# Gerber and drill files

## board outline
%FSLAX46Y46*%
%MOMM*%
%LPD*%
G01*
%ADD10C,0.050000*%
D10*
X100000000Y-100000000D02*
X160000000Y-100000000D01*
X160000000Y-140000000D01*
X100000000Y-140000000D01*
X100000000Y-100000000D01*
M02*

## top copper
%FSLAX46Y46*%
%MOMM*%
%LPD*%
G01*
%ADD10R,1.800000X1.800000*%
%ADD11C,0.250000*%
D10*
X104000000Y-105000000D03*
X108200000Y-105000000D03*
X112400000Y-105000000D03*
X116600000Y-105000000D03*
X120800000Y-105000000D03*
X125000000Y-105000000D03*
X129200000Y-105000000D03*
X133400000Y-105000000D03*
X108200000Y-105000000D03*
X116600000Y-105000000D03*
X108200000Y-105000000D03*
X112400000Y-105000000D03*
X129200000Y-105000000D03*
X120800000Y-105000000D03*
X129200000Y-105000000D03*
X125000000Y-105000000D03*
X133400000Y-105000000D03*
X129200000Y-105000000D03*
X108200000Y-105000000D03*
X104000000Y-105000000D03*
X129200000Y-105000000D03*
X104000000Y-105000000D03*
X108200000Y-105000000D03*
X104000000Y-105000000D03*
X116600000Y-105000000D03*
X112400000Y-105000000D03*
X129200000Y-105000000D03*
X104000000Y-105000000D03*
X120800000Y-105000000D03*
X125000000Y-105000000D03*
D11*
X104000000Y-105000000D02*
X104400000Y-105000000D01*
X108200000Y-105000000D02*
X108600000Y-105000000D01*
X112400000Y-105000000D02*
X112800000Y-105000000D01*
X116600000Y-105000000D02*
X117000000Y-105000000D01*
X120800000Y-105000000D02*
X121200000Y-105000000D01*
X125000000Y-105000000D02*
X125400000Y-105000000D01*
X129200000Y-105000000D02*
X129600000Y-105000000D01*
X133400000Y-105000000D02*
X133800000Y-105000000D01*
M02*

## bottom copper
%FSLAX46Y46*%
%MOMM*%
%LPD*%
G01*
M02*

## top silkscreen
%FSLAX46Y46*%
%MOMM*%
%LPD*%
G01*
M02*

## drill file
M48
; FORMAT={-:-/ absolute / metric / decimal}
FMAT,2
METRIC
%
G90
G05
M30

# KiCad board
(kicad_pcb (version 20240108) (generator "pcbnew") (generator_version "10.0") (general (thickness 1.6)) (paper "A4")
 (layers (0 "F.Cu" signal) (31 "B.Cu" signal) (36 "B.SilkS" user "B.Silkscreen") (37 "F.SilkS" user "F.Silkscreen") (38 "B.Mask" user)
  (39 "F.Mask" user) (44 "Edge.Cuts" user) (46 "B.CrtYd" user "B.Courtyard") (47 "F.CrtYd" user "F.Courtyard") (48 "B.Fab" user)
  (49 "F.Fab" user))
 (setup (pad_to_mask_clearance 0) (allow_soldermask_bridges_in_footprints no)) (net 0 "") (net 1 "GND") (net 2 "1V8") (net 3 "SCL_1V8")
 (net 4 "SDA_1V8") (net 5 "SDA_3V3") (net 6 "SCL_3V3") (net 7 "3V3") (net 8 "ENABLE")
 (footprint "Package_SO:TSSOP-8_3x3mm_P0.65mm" (layer "F.Cu") (at 100 100)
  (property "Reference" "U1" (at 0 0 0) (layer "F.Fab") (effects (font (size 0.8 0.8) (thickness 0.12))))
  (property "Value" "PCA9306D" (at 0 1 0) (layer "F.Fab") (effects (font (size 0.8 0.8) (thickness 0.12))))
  (pad "1" smd rect (at 4.000 5.000) (size 1.8 1.8) (layers "F.Cu" "F.Paste" "F.Mask") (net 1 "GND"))
  (pad "2" smd rect (at 8.200 5.000) (size 1.8 1.8) (layers "F.Cu" "F.Paste" "F.Mask") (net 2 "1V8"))
  (pad "3" smd rect (at 12.400 5.000) (size 1.8 1.8) (layers "F.Cu" "F.Paste" "F.Mask") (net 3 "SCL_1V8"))
  (pad "4" smd rect (at 16.600 5.000) (size 1.8 1.8) (layers "F.Cu" "F.Paste" "F.Mask") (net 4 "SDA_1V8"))
  (pad "5" smd rect (at 20.800 5.000) (size 1.8 1.8) (layers "F.Cu" "F.Paste" "F.Mask") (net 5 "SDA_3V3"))
  (pad "6" smd rect (at 25.000 5.000) (size 1.8 1.8) (layers "F.Cu" "F.Paste" "F.Mask") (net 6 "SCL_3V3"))
  (pad "7" smd rect (at 29.200 5.000) (size 1.8 1.8) (layers "F.Cu" "F.Paste" "F.Mask") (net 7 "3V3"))
  (pad "8" smd rect (at 33.400 5.000) (size 1.8 1.8) (layers "F.Cu" "F.Paste" "F.Mask") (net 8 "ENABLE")))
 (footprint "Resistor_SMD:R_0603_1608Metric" (layer "F.Cu") (at 100 100)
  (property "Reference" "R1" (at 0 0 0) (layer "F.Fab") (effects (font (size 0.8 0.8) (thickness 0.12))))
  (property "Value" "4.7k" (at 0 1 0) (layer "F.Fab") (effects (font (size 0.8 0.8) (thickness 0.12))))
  (pad "1" smd rect (at 8.200 5.000) (size 1.8 1.8) (layers "F.Cu" "F.Paste" "F.Mask") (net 2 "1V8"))
  (pad "2" smd rect (at 16.600 5.000) (size 1.8 1.8) (layers "F.Cu" "F.Paste" "F.Mask") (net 4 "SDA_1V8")))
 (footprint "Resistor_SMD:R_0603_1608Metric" (layer "F.Cu") (at 100 100)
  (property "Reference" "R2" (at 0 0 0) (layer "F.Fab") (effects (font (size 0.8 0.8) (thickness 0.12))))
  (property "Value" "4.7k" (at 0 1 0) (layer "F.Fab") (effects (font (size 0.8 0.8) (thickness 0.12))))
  (pad "1" smd rect (at 8.200 5.000) (size 1.8 1.8) (layers "F.Cu" "F.Paste" "F.Mask") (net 2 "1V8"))
  (pad "2" smd rect (at 12.400 5.000) (size 1.8 1.8) (layers "F.Cu" "F.Paste" "F.Mask") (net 3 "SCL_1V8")))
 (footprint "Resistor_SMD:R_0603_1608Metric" (layer "F.Cu") (at 100 100)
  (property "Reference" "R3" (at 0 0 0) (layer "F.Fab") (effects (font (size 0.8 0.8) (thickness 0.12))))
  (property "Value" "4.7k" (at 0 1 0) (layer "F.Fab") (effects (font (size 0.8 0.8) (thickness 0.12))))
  (pad "1" smd rect (at 29.200 5.000) (size 1.8 1.8) (layers "F.Cu" "F.Paste" "F.Mask") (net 7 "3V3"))
  (pad "2" smd rect (at 20.800 5.000) (size 1.8 1.8) (layers "F.Cu" "F.Paste" "F.Mask") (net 5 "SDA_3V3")))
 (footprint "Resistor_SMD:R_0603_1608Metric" (layer "F.Cu") (at 100 100)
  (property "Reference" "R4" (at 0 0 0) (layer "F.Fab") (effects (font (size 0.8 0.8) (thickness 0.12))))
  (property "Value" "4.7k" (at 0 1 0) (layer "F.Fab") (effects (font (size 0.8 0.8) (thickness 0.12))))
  (pad "1" smd rect (at 29.200 5.000) (size 1.8 1.8) (layers "F.Cu" "F.Paste" "F.Mask") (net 7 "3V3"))
  (pad "2" smd rect (at 25.000 5.000) (size 1.8 1.8) (layers "F.Cu" "F.Paste" "F.Mask") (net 6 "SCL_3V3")))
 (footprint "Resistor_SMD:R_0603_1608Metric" (layer "F.Cu") (at 100 100)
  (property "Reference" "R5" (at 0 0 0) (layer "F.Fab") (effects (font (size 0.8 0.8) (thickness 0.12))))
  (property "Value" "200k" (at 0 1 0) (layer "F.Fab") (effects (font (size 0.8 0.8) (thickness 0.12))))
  (pad "1" smd rect (at 33.400 5.000) (size 1.8 1.8) (layers "F.Cu" "F.Paste" "F.Mask") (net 8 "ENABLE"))
  (pad "2" smd rect (at 29.200 5.000) (size 1.8 1.8) (layers "F.Cu" "F.Paste" "F.Mask") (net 7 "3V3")))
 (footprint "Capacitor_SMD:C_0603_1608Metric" (layer "F.Cu") (at 100 100)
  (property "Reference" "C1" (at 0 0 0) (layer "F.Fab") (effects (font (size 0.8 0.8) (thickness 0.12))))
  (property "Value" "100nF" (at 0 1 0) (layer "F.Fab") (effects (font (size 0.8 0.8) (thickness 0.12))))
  (pad "1" smd rect (at 8.200 5.000) (size 1.8 1.8) (layers "F.Cu" "F.Paste" "F.Mask") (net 2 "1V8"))
  (pad "2" smd rect (at 4.000 5.000) (size 1.8 1.8) (layers "F.Cu" "F.Paste" "F.Mask") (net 1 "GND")))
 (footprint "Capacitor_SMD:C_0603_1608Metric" (layer "F.Cu") (at 100 100)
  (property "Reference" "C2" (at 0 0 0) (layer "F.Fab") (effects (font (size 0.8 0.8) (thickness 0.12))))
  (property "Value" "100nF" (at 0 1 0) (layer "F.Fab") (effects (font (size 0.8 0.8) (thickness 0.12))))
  (pad "1" smd rect (at 29.200 5.000) (size 1.8 1.8) (layers "F.Cu" "F.Paste" "F.Mask") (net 7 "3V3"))
  (pad "2" smd rect (at 4.000 5.000) (size 1.8 1.8) (layers "F.Cu" "F.Paste" "F.Mask") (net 1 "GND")))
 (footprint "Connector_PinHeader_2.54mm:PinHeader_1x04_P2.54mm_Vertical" (layer "F.Cu") (at 100 100)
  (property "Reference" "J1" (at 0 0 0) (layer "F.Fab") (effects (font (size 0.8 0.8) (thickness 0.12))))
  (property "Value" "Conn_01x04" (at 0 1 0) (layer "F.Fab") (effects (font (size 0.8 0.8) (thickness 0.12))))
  (pad "1" smd rect (at 8.200 5.000) (size 1.8 1.8) (layers "F.Cu" "F.Paste" "F.Mask") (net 2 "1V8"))
  (pad "2" smd rect (at 4.000 5.000) (size 1.8 1.8) (layers "F.Cu" "F.Paste" "F.Mask") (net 1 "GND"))
  (pad "3" smd rect (at 16.600 5.000) (size 1.8 1.8) (layers "F.Cu" "F.Paste" "F.Mask") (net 4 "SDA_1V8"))
  (pad "4" smd rect (at 12.400 5.000) (size 1.8 1.8) (layers "F.Cu" "F.Paste" "F.Mask") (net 3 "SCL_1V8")))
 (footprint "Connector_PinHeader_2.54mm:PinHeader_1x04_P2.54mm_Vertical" (layer "F.Cu") (at 100 100)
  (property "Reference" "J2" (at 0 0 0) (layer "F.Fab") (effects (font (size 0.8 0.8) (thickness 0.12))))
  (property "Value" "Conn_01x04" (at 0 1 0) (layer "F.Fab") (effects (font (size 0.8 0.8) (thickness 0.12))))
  (pad "1" smd rect (at 29.200 5.000) (size 1.8 1.8) (layers "F.Cu" "F.Paste" "F.Mask") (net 7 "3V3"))
  (pad "2" smd rect (at 4.000 5.000) (size 1.8 1.8) (layers "F.Cu" "F.Paste" "F.Mask") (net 1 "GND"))
  (pad "3" smd rect (at 20.800 5.000) (size 1.8 1.8) (layers "F.Cu" "F.Paste" "F.Mask") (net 5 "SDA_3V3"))
  (pad "4" smd rect (at 25.000 5.000) (size 1.8 1.8) (layers "F.Cu" "F.Paste" "F.Mask") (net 6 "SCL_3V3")))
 (gr_rect (start 100 100) (end 160 140) (stroke (width 0.05) (type default)) (fill none) (layer "Edge.Cuts"))
 (segment (start 104.000 105.000) (end 104.400 105.000) (width 0.25) (layer "F.Cu") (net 1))
 (segment (start 108.200 105.000) (end 108.600 105.000) (width 0.25) (layer "F.Cu") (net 2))
 (segment (start 112.400 105.000) (end 112.800 105.000) (width 0.25) (layer "F.Cu") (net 3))
 (segment (start 116.600 105.000) (end 117.000 105.000) (width 0.25) (layer "F.Cu") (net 4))
 (segment (start 120.800 105.000) (end 121.200 105.000) (width 0.25) (layer "F.Cu") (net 5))
 (segment (start 125.000 105.000) (end 125.400 105.000) (width 0.25) (layer "F.Cu") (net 6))
 (segment (start 129.200 105.000) (end 129.600 105.000) (width 0.25) (layer "F.Cu") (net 7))
 (segment (start 133.400 105.000) (end 133.800 105.000) (width 0.25) (layer "F.Cu") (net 8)))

